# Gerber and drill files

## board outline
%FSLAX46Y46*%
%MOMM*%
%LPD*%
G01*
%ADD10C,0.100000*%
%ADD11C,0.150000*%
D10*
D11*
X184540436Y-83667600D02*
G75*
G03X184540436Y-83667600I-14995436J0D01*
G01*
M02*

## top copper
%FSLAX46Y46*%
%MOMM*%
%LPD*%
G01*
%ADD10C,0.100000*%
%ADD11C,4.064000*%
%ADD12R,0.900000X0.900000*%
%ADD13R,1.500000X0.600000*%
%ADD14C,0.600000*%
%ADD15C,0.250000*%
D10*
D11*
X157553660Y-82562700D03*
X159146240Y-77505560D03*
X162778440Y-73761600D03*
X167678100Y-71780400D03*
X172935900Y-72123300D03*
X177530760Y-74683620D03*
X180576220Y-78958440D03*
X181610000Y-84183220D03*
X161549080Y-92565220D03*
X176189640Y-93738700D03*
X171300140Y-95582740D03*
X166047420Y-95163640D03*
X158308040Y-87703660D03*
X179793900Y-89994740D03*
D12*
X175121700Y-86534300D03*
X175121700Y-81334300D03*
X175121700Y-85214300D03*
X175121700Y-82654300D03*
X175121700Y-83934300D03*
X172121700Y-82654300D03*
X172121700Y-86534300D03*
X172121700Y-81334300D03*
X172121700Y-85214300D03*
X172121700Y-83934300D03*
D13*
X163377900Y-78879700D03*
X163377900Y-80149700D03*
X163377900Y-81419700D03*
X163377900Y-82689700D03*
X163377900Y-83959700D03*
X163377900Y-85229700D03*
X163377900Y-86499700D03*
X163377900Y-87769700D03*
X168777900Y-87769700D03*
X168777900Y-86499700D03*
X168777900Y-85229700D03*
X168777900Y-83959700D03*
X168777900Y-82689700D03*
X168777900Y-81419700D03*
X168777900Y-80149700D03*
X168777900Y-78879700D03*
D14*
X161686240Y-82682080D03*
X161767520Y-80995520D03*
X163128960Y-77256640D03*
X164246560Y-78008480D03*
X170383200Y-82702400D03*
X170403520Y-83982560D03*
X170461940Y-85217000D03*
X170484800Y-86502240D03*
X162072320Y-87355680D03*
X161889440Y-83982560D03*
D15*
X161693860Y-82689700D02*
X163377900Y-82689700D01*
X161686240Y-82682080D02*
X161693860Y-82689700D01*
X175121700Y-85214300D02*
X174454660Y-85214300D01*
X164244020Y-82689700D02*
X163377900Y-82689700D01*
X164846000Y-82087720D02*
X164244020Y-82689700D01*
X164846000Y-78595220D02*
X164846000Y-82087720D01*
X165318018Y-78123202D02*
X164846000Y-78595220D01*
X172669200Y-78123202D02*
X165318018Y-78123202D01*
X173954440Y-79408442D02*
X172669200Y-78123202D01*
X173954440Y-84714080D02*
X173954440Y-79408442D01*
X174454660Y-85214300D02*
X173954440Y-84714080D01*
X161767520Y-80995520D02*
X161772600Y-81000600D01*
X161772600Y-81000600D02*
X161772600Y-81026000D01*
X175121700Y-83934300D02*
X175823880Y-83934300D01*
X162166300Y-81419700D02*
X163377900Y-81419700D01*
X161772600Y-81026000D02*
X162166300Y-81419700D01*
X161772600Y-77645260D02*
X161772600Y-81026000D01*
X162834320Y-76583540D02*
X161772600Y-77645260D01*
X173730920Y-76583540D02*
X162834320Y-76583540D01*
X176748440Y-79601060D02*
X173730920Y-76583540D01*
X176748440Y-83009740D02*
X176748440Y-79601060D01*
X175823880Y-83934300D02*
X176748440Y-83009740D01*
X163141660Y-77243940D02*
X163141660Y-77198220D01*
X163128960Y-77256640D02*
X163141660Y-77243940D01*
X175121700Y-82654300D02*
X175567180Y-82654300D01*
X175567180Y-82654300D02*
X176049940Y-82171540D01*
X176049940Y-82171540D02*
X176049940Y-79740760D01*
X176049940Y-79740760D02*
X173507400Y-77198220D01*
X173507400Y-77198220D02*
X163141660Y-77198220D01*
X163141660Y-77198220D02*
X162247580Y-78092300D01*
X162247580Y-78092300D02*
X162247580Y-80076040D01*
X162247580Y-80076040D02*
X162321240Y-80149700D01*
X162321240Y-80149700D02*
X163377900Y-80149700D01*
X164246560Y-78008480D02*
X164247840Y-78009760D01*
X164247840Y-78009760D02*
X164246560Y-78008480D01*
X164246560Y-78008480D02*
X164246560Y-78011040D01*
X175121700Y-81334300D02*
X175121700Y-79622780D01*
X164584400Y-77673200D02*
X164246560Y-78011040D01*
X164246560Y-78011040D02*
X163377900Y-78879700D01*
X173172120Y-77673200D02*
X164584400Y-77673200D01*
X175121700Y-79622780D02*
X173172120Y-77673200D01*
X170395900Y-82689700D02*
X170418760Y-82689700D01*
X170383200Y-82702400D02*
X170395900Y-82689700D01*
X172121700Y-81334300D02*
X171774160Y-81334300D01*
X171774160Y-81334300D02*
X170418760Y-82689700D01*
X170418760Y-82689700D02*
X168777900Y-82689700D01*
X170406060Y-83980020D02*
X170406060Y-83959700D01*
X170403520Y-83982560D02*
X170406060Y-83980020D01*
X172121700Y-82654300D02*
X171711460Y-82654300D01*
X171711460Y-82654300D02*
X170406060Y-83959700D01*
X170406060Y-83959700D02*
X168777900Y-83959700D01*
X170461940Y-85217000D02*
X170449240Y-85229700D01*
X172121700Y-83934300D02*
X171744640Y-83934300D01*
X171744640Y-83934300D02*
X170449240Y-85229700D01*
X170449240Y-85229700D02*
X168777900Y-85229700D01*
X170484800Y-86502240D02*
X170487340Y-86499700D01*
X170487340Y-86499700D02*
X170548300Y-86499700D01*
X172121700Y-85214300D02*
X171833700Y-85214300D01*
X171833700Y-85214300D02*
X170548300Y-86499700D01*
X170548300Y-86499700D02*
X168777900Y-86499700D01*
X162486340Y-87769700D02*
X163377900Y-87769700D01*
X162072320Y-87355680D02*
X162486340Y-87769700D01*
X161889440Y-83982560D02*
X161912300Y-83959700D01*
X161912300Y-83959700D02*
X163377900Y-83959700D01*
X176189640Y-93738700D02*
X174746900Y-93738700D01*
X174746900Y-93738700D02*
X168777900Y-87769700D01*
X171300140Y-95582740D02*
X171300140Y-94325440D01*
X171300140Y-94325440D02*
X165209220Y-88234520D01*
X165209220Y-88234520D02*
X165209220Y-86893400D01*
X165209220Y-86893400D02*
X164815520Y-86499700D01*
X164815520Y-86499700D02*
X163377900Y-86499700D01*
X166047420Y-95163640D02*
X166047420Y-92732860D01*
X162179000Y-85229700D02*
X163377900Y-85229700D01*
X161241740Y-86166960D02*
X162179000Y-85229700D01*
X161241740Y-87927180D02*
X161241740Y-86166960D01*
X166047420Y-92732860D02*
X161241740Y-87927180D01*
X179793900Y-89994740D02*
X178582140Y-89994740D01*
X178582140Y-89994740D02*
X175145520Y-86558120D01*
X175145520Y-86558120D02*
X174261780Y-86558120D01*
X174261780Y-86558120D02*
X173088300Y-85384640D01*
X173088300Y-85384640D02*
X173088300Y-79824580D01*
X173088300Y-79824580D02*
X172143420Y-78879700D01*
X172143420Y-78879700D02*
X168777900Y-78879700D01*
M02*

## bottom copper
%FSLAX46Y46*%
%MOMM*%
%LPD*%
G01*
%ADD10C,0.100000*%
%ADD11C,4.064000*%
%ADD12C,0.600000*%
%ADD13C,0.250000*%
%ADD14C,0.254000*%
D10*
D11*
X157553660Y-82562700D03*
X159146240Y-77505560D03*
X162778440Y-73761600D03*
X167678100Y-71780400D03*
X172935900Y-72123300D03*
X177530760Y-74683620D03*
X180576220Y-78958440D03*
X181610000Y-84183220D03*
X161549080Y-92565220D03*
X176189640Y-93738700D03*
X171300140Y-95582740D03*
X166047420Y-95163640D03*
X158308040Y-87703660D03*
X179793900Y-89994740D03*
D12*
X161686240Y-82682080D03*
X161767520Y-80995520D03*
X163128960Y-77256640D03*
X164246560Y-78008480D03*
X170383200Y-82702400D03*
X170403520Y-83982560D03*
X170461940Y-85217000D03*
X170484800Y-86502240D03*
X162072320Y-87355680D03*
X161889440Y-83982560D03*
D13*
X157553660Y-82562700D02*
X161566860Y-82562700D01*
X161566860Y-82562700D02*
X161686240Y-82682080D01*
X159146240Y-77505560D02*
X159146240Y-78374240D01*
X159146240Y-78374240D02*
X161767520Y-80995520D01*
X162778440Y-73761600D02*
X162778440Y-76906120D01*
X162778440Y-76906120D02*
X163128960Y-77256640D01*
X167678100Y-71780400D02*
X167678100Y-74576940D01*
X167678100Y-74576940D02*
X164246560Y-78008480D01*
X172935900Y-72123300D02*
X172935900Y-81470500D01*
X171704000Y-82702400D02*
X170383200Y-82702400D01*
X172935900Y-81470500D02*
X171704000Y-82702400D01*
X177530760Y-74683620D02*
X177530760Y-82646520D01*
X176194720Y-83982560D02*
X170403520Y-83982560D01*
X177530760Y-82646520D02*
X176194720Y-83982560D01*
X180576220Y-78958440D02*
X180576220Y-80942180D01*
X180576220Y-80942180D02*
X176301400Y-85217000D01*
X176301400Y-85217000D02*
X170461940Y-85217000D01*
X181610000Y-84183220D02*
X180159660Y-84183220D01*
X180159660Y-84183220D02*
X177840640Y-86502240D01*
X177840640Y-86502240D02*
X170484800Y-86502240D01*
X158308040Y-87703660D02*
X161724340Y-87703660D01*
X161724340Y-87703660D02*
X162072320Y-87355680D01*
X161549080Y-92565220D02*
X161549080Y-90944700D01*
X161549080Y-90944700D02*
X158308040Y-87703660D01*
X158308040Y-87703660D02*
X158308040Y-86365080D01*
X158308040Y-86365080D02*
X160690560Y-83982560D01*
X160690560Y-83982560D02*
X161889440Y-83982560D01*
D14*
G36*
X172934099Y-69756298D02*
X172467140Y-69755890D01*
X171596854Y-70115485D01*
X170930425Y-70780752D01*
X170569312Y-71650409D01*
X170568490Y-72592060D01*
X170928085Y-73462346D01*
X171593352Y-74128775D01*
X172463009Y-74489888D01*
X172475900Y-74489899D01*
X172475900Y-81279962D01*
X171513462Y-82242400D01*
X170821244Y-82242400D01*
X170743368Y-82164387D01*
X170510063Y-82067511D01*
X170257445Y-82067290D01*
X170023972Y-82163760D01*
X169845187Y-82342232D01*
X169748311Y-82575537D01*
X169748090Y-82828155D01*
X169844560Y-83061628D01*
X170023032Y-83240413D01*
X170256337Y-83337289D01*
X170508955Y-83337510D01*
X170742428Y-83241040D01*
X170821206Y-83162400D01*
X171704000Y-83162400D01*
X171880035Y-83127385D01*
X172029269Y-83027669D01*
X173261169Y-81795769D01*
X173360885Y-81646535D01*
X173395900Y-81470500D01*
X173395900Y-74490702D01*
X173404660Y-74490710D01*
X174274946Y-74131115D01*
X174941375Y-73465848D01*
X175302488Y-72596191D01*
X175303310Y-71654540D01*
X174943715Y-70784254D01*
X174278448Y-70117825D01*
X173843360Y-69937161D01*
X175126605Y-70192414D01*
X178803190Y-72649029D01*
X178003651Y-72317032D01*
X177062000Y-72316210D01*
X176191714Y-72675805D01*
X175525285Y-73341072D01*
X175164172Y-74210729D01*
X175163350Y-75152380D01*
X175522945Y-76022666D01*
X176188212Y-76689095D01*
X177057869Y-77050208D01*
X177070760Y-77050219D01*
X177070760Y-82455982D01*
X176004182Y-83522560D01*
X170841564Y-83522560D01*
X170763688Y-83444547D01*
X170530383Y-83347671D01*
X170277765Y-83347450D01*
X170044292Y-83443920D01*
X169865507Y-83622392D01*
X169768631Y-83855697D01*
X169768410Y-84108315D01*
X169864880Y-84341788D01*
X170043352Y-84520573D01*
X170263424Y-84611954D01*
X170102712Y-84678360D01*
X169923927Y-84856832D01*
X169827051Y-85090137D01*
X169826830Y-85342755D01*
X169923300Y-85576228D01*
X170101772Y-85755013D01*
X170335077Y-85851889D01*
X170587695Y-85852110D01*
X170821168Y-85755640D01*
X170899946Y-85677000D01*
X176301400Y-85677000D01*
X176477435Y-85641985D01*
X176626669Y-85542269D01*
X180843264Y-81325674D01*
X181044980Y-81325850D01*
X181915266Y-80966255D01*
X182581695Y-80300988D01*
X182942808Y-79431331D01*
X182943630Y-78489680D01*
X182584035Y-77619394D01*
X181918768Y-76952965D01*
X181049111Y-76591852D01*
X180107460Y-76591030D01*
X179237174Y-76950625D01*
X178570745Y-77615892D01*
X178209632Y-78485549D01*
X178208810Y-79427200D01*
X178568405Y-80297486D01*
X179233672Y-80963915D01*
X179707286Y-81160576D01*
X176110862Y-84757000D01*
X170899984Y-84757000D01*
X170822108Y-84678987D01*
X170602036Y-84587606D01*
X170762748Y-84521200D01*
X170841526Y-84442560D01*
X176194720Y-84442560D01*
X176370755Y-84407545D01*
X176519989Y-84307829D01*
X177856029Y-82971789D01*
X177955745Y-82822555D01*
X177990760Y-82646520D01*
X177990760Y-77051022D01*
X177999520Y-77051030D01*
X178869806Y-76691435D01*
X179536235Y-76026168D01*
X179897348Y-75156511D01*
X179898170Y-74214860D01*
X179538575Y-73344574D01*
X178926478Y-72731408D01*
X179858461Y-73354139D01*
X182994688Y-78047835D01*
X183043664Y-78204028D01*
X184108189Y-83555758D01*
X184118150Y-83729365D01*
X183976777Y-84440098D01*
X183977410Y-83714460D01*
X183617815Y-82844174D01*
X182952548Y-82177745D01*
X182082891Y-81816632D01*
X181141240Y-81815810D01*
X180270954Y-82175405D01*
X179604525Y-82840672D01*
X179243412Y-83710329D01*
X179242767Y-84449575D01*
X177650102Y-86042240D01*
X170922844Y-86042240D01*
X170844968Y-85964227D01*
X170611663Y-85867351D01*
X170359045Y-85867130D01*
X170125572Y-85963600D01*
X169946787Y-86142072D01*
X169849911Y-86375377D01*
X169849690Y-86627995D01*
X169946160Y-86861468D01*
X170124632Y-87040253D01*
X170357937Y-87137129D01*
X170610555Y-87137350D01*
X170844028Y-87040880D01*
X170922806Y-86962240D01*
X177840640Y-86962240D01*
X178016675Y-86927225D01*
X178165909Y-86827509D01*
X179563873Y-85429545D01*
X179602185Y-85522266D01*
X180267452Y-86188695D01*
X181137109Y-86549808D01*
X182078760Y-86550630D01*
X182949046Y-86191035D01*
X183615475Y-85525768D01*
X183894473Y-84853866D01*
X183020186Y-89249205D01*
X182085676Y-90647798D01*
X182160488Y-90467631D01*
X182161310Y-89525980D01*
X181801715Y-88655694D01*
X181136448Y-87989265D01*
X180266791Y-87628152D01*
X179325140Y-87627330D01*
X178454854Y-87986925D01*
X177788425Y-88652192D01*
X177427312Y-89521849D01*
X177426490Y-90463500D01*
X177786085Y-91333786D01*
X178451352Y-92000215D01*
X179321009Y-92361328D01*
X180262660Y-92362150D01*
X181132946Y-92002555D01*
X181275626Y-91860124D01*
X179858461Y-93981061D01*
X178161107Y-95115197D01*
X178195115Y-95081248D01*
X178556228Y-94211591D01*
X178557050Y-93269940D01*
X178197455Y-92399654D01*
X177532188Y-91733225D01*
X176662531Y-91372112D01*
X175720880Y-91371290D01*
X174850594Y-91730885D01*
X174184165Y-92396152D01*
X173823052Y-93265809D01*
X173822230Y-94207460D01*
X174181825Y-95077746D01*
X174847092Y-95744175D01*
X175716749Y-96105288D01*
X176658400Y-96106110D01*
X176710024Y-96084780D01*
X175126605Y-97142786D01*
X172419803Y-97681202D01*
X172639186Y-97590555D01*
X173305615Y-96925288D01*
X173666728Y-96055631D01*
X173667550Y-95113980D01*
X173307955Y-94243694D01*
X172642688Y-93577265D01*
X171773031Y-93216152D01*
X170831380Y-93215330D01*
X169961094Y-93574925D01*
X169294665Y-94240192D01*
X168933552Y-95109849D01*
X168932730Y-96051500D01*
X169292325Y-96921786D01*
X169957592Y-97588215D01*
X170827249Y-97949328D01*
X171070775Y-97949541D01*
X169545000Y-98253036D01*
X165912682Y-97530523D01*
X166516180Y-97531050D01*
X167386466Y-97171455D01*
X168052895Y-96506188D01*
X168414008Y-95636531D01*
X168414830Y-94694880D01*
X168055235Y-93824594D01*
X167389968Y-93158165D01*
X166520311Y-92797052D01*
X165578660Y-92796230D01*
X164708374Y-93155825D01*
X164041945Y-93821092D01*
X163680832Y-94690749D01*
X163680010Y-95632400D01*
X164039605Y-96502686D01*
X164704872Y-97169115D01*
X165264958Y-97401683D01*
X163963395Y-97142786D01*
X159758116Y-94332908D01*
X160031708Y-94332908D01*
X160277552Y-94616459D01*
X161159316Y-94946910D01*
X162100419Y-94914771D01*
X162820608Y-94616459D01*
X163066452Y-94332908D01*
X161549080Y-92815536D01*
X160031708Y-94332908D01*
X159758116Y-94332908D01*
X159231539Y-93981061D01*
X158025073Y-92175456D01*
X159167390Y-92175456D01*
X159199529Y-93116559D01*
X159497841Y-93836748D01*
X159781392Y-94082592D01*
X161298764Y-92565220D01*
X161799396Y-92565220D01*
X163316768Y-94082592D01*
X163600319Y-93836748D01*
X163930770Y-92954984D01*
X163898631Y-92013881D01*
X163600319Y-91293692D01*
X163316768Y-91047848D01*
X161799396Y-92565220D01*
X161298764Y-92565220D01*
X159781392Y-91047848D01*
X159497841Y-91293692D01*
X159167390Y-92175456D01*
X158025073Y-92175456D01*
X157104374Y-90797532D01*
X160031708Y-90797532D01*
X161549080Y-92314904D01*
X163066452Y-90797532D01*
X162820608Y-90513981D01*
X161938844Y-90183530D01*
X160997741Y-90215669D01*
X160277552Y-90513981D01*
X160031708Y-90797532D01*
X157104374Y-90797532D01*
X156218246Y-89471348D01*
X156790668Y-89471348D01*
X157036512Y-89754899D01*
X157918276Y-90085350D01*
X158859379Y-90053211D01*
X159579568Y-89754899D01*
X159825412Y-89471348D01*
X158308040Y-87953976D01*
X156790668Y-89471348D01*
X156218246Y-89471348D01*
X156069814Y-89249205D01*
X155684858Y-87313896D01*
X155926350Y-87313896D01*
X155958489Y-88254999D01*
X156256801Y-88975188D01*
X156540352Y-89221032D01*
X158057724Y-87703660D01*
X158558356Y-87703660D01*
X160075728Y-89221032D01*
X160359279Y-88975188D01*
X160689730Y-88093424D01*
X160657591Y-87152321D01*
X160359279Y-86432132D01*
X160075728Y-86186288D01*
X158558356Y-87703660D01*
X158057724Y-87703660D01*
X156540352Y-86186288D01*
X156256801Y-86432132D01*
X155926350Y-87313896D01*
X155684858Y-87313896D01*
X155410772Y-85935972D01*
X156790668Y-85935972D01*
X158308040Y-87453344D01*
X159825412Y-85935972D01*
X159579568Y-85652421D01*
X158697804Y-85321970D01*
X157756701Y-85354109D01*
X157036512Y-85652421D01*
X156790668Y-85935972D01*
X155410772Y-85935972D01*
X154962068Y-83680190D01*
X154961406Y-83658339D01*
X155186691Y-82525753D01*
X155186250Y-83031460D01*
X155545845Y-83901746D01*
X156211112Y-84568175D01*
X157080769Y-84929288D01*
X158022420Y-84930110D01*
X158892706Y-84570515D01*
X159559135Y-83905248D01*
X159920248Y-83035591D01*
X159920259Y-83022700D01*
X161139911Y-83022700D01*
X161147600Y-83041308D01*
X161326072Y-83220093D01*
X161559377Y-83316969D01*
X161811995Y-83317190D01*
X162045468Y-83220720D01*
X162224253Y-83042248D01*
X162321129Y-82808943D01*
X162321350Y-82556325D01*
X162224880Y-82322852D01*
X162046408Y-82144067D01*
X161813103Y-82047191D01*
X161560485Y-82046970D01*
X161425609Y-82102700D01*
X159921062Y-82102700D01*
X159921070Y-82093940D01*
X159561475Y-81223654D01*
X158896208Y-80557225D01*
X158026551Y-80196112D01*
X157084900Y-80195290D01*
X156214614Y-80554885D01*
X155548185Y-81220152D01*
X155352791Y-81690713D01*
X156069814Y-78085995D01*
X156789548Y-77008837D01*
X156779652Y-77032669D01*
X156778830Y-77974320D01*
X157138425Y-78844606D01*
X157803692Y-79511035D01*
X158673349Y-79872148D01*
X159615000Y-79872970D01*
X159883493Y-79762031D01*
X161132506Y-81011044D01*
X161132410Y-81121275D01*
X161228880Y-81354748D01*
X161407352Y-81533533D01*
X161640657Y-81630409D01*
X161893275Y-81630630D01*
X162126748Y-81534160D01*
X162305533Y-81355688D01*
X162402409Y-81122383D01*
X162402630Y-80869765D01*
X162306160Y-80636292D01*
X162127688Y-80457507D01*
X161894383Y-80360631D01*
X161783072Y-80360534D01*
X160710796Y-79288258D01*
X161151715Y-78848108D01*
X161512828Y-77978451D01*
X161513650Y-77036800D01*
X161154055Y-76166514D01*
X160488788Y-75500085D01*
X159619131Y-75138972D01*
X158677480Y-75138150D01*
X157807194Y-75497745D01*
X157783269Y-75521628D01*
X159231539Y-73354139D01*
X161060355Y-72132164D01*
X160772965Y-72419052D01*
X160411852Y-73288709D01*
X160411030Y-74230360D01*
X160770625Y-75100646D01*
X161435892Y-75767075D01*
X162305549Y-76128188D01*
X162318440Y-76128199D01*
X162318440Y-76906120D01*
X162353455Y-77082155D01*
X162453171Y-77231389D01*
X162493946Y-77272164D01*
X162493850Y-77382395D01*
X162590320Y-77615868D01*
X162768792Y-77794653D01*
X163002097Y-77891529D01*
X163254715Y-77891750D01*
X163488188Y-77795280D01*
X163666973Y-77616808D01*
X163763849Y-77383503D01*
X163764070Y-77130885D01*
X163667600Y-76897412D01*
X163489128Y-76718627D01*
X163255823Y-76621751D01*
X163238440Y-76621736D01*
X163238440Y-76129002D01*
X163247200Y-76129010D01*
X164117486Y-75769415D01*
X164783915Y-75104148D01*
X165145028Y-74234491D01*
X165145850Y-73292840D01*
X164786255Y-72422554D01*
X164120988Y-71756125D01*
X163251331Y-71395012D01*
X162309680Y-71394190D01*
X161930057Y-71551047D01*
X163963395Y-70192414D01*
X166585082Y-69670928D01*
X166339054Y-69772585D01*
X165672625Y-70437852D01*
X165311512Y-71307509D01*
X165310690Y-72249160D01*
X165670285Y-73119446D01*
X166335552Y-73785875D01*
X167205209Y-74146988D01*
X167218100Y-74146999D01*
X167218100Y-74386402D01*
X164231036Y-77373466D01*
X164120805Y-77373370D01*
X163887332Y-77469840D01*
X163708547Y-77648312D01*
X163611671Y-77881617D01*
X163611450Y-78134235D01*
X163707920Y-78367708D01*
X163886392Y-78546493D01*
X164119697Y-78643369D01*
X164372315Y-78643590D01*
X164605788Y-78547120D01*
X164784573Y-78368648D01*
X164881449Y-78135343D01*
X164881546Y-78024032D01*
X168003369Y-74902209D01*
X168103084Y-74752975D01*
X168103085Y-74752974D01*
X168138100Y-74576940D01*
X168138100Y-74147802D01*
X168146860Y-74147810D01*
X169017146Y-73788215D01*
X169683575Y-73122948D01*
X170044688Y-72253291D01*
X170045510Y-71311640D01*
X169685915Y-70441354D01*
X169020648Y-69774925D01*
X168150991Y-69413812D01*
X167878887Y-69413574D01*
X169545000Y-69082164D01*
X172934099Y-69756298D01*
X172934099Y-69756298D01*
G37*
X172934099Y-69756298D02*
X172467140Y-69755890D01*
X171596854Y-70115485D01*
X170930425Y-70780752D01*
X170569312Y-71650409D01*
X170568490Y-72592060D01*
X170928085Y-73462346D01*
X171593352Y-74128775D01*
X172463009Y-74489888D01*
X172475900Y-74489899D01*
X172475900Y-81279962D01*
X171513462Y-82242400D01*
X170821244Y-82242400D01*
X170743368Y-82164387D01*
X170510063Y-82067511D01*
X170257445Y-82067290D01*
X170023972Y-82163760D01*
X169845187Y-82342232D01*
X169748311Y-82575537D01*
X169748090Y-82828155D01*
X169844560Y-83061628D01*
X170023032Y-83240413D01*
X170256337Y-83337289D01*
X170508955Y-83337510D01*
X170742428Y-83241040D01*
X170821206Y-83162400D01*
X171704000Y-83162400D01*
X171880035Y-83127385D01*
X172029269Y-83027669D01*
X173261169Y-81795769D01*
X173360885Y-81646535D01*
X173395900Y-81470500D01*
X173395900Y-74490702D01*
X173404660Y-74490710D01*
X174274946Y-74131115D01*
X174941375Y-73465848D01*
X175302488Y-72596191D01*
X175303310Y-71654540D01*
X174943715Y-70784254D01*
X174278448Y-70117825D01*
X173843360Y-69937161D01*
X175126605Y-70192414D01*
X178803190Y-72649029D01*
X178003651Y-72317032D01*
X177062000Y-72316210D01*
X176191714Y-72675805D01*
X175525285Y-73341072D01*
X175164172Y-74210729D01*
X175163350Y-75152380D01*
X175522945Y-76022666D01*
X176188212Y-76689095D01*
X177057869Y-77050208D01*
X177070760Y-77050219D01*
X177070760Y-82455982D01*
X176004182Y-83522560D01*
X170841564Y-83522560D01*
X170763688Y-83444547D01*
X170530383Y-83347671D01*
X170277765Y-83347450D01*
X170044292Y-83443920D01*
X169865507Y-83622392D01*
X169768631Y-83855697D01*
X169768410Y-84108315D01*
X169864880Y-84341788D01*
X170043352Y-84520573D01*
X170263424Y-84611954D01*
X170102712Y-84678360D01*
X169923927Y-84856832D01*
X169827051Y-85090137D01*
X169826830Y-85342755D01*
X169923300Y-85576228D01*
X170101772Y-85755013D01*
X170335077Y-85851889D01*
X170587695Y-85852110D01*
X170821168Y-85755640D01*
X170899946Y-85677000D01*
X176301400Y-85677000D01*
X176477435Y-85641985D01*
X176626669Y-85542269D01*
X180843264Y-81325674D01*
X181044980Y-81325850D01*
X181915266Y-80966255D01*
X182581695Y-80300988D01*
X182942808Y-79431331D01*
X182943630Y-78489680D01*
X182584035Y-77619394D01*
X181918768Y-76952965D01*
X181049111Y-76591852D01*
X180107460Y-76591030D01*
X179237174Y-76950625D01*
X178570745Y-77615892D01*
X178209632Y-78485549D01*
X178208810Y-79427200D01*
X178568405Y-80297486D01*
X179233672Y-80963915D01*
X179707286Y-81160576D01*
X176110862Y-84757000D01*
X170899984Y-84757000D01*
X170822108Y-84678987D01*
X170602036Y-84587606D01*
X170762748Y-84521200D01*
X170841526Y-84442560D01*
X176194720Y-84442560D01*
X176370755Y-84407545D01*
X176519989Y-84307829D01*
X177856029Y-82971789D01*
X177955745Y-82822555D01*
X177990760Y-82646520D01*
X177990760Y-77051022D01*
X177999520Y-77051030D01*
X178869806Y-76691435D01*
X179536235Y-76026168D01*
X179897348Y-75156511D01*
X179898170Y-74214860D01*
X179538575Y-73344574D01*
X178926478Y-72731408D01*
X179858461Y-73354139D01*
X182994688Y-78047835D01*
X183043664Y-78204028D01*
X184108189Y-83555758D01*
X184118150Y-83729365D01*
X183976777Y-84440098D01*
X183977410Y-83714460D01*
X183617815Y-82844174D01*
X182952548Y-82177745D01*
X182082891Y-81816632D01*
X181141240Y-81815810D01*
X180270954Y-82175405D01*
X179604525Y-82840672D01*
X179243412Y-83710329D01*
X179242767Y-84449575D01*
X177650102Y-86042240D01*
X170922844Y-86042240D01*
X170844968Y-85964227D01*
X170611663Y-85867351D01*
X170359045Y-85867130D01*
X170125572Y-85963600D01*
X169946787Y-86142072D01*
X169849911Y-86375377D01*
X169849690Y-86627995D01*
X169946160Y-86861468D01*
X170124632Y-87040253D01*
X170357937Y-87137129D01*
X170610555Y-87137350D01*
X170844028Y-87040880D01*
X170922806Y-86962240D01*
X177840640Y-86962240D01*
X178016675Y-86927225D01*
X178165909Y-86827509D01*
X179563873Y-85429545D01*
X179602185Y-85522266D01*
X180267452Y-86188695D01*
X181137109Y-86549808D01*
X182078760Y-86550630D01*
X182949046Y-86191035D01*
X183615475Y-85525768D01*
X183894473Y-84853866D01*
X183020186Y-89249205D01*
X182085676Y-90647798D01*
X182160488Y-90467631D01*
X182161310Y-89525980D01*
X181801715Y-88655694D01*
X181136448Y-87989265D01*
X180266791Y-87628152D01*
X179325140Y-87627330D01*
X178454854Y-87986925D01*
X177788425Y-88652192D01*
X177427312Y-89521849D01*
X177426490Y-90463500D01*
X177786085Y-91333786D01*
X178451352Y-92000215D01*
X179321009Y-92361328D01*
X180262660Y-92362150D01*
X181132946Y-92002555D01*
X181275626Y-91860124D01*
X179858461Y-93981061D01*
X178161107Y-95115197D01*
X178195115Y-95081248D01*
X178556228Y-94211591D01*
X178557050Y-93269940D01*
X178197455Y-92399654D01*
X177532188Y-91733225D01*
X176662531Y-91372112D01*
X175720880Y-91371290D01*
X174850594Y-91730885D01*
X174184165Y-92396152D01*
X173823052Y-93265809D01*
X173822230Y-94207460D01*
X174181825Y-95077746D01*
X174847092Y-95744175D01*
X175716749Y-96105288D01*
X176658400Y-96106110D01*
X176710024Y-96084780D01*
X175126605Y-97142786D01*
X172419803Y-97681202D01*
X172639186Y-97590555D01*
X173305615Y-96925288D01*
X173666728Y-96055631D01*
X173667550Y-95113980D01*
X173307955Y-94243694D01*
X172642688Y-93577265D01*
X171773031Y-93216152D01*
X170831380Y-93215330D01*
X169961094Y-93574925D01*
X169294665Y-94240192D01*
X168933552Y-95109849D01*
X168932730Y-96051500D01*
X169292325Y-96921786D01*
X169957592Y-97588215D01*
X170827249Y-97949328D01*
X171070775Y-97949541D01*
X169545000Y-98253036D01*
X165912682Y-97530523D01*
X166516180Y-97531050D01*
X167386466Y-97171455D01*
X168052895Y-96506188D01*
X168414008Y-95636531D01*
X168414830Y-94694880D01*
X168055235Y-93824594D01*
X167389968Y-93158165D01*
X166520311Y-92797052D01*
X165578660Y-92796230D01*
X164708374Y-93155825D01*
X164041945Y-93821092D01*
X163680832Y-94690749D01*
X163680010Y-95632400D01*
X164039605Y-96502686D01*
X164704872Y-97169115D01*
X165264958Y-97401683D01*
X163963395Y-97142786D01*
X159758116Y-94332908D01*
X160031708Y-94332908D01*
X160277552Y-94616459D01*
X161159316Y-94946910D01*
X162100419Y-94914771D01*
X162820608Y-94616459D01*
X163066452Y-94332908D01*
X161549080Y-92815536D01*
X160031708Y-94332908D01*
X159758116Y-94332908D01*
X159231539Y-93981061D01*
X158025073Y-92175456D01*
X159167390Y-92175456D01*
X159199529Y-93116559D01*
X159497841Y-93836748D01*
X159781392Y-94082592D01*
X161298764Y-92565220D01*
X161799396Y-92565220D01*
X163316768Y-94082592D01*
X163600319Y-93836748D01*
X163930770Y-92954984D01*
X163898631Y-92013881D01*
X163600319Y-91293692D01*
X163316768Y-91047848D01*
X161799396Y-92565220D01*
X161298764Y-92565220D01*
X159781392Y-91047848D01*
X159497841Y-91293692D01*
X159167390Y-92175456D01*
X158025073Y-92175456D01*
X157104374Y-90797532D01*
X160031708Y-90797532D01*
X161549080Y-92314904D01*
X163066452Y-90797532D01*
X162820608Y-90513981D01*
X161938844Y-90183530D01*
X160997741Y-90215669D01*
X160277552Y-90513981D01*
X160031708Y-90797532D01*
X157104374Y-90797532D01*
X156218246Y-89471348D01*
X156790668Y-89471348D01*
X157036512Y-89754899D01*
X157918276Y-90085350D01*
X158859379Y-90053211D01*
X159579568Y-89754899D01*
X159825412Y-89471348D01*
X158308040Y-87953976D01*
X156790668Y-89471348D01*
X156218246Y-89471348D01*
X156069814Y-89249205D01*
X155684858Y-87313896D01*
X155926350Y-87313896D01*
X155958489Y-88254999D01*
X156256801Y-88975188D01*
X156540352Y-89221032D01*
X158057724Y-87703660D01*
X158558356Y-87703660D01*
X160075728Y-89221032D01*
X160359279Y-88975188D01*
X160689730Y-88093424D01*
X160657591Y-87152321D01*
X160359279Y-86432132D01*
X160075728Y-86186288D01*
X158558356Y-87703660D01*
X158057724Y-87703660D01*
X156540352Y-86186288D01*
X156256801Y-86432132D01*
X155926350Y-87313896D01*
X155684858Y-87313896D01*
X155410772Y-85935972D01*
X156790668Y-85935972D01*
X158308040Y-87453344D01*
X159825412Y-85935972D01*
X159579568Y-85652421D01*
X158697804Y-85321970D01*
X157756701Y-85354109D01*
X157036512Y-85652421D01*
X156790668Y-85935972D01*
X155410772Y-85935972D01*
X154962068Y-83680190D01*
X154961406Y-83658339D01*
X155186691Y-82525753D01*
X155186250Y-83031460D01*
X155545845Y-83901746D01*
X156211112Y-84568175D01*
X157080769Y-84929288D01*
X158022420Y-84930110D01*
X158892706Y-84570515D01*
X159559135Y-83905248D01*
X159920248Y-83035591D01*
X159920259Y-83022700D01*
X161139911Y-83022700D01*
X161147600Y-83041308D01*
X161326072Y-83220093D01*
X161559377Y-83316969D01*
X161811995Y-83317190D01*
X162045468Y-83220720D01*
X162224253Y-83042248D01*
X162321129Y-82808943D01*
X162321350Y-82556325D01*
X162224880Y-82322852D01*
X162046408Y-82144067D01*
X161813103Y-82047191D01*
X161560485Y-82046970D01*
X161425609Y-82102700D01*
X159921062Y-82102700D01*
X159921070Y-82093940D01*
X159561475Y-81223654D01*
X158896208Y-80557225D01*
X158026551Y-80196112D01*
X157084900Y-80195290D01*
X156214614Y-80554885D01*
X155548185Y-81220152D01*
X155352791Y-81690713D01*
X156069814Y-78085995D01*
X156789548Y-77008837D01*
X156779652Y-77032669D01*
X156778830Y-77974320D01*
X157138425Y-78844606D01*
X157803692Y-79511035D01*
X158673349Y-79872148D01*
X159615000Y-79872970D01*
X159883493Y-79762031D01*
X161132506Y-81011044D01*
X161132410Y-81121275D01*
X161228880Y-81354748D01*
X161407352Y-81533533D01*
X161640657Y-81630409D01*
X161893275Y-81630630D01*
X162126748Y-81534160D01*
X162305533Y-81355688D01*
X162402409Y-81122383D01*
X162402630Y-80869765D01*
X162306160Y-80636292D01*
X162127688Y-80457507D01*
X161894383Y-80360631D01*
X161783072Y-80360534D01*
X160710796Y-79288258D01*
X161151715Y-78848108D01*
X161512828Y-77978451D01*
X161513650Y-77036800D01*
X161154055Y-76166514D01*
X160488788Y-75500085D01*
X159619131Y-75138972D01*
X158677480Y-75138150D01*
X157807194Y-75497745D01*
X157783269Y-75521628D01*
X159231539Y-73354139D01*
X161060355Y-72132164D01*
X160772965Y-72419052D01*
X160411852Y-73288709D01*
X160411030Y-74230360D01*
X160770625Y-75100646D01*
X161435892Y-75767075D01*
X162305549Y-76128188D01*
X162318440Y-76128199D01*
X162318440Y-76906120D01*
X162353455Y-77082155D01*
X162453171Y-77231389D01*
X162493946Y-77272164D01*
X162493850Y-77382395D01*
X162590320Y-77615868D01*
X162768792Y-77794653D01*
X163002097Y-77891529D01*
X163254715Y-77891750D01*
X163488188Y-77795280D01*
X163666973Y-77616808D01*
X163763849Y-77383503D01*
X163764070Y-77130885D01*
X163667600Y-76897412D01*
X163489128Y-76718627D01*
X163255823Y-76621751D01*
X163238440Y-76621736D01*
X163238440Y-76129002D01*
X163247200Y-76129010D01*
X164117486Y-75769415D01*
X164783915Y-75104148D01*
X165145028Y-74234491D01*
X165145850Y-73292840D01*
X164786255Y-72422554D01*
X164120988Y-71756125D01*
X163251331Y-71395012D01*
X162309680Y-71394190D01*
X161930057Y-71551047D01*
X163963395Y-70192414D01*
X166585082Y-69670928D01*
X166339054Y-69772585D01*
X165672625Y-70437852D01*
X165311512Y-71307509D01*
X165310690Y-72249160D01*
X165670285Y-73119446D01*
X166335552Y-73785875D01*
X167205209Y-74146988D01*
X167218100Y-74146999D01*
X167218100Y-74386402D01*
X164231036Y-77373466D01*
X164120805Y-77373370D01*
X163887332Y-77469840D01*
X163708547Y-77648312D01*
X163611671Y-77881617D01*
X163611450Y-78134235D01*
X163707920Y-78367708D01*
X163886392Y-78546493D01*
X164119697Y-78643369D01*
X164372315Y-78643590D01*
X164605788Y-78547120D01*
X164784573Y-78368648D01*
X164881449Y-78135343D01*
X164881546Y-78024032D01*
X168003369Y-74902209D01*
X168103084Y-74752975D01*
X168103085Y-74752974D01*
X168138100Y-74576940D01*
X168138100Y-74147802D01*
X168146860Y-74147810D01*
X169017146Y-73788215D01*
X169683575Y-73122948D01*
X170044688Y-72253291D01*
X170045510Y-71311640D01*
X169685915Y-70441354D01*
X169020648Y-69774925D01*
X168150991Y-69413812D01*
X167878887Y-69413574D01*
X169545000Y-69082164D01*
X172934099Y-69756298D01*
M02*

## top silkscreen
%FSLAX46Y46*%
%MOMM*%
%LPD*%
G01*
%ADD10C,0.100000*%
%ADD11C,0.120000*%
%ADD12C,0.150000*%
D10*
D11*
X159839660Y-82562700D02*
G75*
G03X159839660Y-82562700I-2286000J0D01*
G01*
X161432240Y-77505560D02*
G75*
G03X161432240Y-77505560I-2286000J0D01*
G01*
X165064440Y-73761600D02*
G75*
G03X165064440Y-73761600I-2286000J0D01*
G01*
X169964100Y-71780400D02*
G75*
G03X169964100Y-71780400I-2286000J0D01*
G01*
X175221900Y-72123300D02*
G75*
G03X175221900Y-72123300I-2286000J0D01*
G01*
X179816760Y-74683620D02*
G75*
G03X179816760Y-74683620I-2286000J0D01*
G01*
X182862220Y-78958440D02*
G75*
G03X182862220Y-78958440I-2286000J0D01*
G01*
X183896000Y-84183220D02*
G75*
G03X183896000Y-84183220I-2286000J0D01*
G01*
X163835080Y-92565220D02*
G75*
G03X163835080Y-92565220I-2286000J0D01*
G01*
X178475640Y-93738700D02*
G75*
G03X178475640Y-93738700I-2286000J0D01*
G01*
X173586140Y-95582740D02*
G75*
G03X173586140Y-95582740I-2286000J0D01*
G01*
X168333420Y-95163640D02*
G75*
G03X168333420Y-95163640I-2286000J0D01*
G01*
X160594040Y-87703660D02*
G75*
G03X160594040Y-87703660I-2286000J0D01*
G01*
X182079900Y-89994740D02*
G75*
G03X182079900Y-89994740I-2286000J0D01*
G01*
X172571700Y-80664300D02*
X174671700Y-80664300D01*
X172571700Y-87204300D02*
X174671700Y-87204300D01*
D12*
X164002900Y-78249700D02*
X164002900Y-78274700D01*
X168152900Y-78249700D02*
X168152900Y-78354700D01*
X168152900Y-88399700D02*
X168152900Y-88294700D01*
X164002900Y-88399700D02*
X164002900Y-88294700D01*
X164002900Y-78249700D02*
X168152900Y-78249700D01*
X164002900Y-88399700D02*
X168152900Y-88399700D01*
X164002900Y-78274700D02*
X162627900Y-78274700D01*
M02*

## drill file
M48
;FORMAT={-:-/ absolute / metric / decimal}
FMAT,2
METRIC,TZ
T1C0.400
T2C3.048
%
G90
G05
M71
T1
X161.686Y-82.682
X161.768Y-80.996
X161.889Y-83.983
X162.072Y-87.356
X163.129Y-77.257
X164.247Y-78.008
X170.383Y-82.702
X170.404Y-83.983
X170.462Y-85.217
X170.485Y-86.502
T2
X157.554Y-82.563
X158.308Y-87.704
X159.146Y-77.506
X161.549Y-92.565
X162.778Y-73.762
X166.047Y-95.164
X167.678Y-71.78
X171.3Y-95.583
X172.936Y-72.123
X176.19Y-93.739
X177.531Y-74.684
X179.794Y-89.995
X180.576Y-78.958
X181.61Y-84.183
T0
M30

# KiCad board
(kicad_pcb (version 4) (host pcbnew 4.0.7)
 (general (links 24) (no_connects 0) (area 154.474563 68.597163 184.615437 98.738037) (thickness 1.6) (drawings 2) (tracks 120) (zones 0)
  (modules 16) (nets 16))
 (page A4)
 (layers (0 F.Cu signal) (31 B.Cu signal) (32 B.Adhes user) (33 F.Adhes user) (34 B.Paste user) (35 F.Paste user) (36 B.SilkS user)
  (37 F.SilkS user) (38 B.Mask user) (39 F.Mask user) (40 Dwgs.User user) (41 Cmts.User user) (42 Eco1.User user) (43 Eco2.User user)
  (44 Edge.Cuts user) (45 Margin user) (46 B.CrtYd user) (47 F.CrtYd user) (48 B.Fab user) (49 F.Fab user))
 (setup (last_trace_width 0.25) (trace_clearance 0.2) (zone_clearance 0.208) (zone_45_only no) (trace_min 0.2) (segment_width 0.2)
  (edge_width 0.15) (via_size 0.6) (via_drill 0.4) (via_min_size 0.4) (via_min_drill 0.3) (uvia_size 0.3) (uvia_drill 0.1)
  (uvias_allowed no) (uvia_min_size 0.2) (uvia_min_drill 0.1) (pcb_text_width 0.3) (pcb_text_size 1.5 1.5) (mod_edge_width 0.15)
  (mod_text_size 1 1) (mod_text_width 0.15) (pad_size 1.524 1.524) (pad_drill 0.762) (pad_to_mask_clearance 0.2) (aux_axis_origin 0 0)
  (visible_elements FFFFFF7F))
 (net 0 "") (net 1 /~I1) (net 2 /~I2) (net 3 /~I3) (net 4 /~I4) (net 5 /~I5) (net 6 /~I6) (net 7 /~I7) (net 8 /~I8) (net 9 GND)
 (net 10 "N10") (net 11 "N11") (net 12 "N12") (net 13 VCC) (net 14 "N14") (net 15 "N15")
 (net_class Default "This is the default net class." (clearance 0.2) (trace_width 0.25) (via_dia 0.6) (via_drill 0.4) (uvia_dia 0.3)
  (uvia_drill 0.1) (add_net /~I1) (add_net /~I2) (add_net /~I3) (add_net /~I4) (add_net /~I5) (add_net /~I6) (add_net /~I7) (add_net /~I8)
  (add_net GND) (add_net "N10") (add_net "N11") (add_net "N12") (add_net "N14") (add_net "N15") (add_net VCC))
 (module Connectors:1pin (layer F.Cu) (at 157.55366 82.5627)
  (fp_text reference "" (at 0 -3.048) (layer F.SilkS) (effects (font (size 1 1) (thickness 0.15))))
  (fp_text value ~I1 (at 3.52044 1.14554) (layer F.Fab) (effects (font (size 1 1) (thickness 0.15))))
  (fp_circle (center 0 0) (end 0 -2.286) (layer F.SilkS) (width 0.12))
  (pad 1 thru_hole circle (at 0 0) (size 4.064 4.064) (drill 3.048) (layers *.Cu *.Mask) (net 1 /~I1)))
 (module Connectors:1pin (layer F.Cu) (at 159.14624 77.50556)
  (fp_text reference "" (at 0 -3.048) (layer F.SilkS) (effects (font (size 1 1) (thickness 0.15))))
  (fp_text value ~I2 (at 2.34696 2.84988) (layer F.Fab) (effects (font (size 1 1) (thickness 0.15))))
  (fp_circle (center 0 0) (end 0 -2.286) (layer F.SilkS) (width 0.12))
  (pad 1 thru_hole circle (at 0 0) (size 4.064 4.064) (drill 3.048) (layers *.Cu *.Mask) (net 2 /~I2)))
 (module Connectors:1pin (layer F.Cu) (at 162.77844 73.7616)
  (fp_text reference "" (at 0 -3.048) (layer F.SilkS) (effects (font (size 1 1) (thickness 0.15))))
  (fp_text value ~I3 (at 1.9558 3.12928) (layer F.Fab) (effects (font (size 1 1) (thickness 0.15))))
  (fp_circle (center 0 0) (end 0 -2.286) (layer F.SilkS) (width 0.12))
  (pad 1 thru_hole circle (at 0 0) (size 4.064 4.064) (drill 3.048) (layers *.Cu *.Mask) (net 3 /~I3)))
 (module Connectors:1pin (layer F.Cu) (at 167.6781 71.7804)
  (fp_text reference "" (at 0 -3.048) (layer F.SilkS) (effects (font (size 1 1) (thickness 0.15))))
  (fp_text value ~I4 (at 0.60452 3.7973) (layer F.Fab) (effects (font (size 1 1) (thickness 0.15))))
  (fp_circle (center 0 0) (end 0 -2.286) (layer F.SilkS) (width 0.12))
  (pad 1 thru_hole circle (at 0 0) (size 4.064 4.064) (drill 3.048) (layers *.Cu *.Mask) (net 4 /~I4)))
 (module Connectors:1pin (layer F.Cu) (at 172.9359 72.1233)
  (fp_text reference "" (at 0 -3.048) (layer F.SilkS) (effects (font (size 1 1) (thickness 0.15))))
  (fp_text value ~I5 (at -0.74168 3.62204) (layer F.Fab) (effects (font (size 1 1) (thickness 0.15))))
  (fp_circle (center 0 0) (end 0 -2.286) (layer F.SilkS) (width 0.12))
  (pad 1 thru_hole circle (at 0 0) (size 4.064 4.064) (drill 3.048) (layers *.Cu *.Mask) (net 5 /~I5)))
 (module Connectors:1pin (layer F.Cu) (at 177.53076 74.68362)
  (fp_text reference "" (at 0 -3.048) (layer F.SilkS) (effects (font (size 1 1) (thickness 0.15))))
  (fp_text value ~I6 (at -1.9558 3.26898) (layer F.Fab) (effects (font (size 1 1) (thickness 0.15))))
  (fp_circle (center 0 0) (end 0 -2.286) (layer F.SilkS) (width 0.12))
  (pad 1 thru_hole circle (at 0 0) (size 4.064 4.064) (drill 3.048) (layers *.Cu *.Mask) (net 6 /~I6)))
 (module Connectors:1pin (layer F.Cu) (at 180.57622 78.95844)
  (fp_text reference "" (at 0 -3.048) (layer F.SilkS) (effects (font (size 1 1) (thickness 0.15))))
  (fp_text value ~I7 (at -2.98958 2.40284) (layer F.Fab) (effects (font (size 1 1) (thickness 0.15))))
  (fp_circle (center 0 0) (end 0 -2.286) (layer F.SilkS) (width 0.12))
  (pad 1 thru_hole circle (at 0 0) (size 4.064 4.064) (drill 3.048) (layers *.Cu *.Mask) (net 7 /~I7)))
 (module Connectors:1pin (layer F.Cu) (at 181.61 84.18322)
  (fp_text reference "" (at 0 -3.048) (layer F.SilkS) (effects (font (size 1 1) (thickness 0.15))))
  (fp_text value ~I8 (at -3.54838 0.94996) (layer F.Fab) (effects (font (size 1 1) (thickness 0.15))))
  (fp_circle (center 0 0) (end 0 -2.286) (layer F.SilkS) (width 0.12))
  (pad 1 thru_hole circle (at 0 0) (size 4.064 4.064) (drill 3.048) (layers *.Cu *.Mask) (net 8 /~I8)))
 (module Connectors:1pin (layer F.Cu) (at 161.54908 92.56522)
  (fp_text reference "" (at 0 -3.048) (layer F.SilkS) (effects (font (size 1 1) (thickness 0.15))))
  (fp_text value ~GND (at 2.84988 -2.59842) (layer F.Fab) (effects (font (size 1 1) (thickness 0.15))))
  (fp_circle (center 0 0) (end 0 -2.286) (layer F.SilkS) (width 0.12))
  (pad 1 thru_hole circle (at 0 0) (size 4.064 4.064) (drill 3.048) (layers *.Cu *.Mask) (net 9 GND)))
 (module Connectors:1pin (layer F.Cu) (at 176.18964 93.7387)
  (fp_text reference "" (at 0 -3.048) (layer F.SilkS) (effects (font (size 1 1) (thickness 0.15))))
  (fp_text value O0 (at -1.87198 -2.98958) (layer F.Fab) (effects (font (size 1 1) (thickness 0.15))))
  (fp_circle (center 0 0) (end 0 -2.286) (layer F.SilkS) (width 0.12))
  (pad 1 thru_hole circle (at 0 0) (size 4.064 4.064) (drill 3.048) (layers *.Cu *.Mask) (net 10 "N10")))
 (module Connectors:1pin (layer F.Cu) (at 171.30014 95.58274)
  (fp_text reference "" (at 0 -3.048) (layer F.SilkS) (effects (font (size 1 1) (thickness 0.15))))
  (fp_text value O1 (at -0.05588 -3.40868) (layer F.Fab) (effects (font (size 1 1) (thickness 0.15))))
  (fp_circle (center 0 0) (end 0 -2.286) (layer F.SilkS) (width 0.12))
  (pad 1 thru_hole circle (at 0 0) (size 4.064 4.064) (drill 3.048) (layers *.Cu *.Mask) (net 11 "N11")))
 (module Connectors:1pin (layer F.Cu) (at 166.04742 95.16364)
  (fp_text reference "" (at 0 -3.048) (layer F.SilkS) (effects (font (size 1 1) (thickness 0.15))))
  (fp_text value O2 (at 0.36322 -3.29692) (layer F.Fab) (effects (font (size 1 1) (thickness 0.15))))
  (fp_circle (center 0 0) (end 0 -2.286) (layer F.SilkS) (width 0.12))
  (pad 1 thru_hole circle (at 0 0) (size 4.064 4.064) (drill 3.048) (layers *.Cu *.Mask) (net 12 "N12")))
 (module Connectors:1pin (layer F.Cu) (at 158.30804 87.70366)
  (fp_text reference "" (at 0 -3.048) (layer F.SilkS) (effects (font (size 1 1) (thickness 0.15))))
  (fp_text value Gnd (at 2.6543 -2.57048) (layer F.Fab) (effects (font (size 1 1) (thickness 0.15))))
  (fp_circle (center 0 0) (end 0 -2.286) (layer F.SilkS) (width 0.12))
  (pad 1 thru_hole circle (at 0 0) (size 4.064 4.064) (drill 3.048) (layers *.Cu *.Mask) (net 9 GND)))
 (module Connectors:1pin (layer F.Cu) (at 179.7939 89.99474)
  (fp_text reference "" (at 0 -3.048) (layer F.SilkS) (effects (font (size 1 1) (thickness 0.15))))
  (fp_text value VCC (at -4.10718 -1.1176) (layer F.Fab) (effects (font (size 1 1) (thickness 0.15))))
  (fp_circle (center 0 0) (end 0 -2.286) (layer F.SilkS) (width 0.12))
  (pad 1 thru_hole circle (at 0 0) (size 4.064 4.064) (drill 3.048) (layers *.Cu *.Mask) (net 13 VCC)))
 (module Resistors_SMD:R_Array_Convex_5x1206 (layer F.Cu) (at 173.6217 83.9343 180)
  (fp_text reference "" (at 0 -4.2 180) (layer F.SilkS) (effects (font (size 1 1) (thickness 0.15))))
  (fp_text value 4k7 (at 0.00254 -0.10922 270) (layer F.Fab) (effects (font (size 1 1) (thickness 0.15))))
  (fp_line (start 1.05 3.27) (end -1.05 3.27) (layer F.SilkS) (width 0.12))
  (fp_line (start 1.05 -3.27) (end -1.05 -3.27) (layer F.SilkS) (width 0.12))
  (pad 1 smd rect (at -1.5 -2.6 180) (size 0.9 0.9) (layers F.Cu F.Paste F.Mask) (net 13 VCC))
  (pad 5 smd rect (at -1.5 2.6 180) (size 0.9 0.9) (layers F.Cu F.Paste F.Mask) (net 4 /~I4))
  (pad 2 smd rect (at -1.5 -1.28 180) (size 0.9 0.9) (layers F.Cu F.Paste F.Mask) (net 1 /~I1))
  (pad 4 smd rect (at -1.5 1.28 180) (size 0.9 0.9) (layers F.Cu F.Paste F.Mask) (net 3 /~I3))
  (pad 3 smd rect (at -1.5 0 180) (size 0.9 0.9) (layers F.Cu F.Paste F.Mask) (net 2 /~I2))
  (pad 7 smd rect (at 1.5 1.28 180) (size 0.9 0.9) (layers F.Cu F.Paste F.Mask) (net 6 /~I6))
  (pad 10 smd rect (at 1.5 -2.6 180) (size 0.9 0.9) (layers F.Cu F.Paste F.Mask))
  (pad 6 smd rect (at 1.5 2.6 180) (size 0.9 0.9) (layers F.Cu F.Paste F.Mask) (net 5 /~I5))
  (pad 9 smd rect (at 1.5 -1.28 180) (size 0.9 0.9) (layers F.Cu F.Paste F.Mask) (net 8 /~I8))
  (pad 8 smd rect (at 1.5 0 180) (size 0.9 0.9) (layers F.Cu F.Paste F.Mask) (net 7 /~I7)))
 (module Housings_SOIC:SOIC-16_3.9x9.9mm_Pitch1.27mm (layer F.Cu) (at 166.0779 83.3247)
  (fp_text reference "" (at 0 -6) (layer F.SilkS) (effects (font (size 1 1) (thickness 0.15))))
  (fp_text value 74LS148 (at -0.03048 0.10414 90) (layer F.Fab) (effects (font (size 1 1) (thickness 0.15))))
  (fp_line (start -2.075 -5.075) (end -2.075 -5.05) (layer F.SilkS) (width 0.15))
  (fp_line (start 2.075 -5.075) (end 2.075 -4.97) (layer F.SilkS) (width 0.15))
  (fp_line (start 2.075 5.075) (end 2.075 4.97) (layer F.SilkS) (width 0.15))
  (fp_line (start -2.075 5.075) (end -2.075 4.97) (layer F.SilkS) (width 0.15))
  (fp_line (start -2.075 -5.075) (end 2.075 -5.075) (layer F.SilkS) (width 0.15))
  (fp_line (start -2.075 5.075) (end 2.075 5.075) (layer F.SilkS) (width 0.15))
  (fp_line (start -2.075 -5.05) (end -3.45 -5.05) (layer F.SilkS) (width 0.15))
  (pad 1 smd rect (at -2.7 -4.445) (size 1.5 0.6) (layers F.Cu F.Paste F.Mask) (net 4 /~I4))
  (pad 2 smd rect (at -2.7 -3.175) (size 1.5 0.6) (layers F.Cu F.Paste F.Mask) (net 3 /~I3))
  (pad 3 smd rect (at -2.7 -1.905) (size 1.5 0.6) (layers F.Cu F.Paste F.Mask) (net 2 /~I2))
  (pad 4 smd rect (at -2.7 -0.635) (size 1.5 0.6) (layers F.Cu F.Paste F.Mask) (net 1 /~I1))
  (pad 5 smd rect (at -2.7 0.635) (size 1.5 0.6) (layers F.Cu F.Paste F.Mask) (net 9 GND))
  (pad 6 smd rect (at -2.7 1.905) (size 1.5 0.6) (layers F.Cu F.Paste F.Mask) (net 12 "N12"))
  (pad 7 smd rect (at -2.7 3.175) (size 1.5 0.6) (layers F.Cu F.Paste F.Mask) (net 11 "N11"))
  (pad 8 smd rect (at -2.7 4.445) (size 1.5 0.6) (layers F.Cu F.Paste F.Mask) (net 9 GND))
  (pad 9 smd rect (at 2.7 4.445) (size 1.5 0.6) (layers F.Cu F.Paste F.Mask) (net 10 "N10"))
  (pad 10 smd rect (at 2.7 3.175) (size 1.5 0.6) (layers F.Cu F.Paste F.Mask) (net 8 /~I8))
  (pad 11 smd rect (at 2.7 1.905) (size 1.5 0.6) (layers F.Cu F.Paste F.Mask) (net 7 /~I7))
  (pad 12 smd rect (at 2.7 0.635) (size 1.5 0.6) (layers F.Cu F.Paste F.Mask) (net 6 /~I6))
  (pad 13 smd rect (at 2.7 -0.635) (size 1.5 0.6) (layers F.Cu F.Paste F.Mask) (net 5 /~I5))
  (pad 14 smd rect (at 2.7 -1.905) (size 1.5 0.6) (layers F.Cu F.Paste F.Mask) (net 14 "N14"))
  (pad 15 smd rect (at 2.7 -3.175) (size 1.5 0.6) (layers F.Cu F.Paste F.Mask) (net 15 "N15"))
  (pad 16 smd rect (at 2.7 -4.445) (size 1.5 0.6) (layers F.Cu F.Paste F.Mask) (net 13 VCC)))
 (gr_circle (center 169.545 83.6676) (end 180.6321 93.7641) (layer Edge.Cuts) (width 0.15))
 (segment (start 157.55366 82.5627) (end 161.56686 82.5627) (width 0.25) (layer B.Cu) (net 1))
 (segment (start 161.69386 82.6897) (end 163.3779 82.6897) (width 0.25) (layer F.Cu) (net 1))
 (segment (start 161.68624 82.68208) (end 161.69386 82.6897) (width 0.25) (layer F.Cu) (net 1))
 (via (at 161.68624 82.68208) (size 0.6) (drill 0.4) (layers F.Cu B.Cu) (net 1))
 (segment (start 161.56686 82.5627) (end 161.68624 82.68208) (width 0.25) (layer B.Cu) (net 1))
 (segment (start 175.1217 85.2143) (end 174.45466 85.2143) (width 0.25) (layer F.Cu) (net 1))
 (segment (start 164.24402 82.6897) (end 163.3779 82.6897) (width 0.25) (layer F.Cu) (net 1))
 (segment (start 164.846 82.08772) (end 164.24402 82.6897) (width 0.25) (layer F.Cu) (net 1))
 (segment (start 164.846 78.59522) (end 164.846 82.08772) (width 0.25) (layer F.Cu) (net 1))
 (segment (start 165.318018 78.123202) (end 164.846 78.59522) (width 0.25) (layer F.Cu) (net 1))
 (segment (start 172.6692 78.123202) (end 165.318018 78.123202) (width 0.25) (layer F.Cu) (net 1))
 (segment (start 173.95444 79.408442) (end 172.6692 78.123202) (width 0.25) (layer F.Cu) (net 1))
 (segment (start 173.95444 84.71408) (end 173.95444 79.408442) (width 0.25) (layer F.Cu) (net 1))
 (segment (start 174.45466 85.2143) (end 173.95444 84.71408) (width 0.25) (layer F.Cu) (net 1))
 (segment (start 159.14624 77.50556) (end 159.14624 78.37424) (width 0.25) (layer B.Cu) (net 2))
 (segment (start 159.14624 78.37424) (end 161.76752 80.99552) (width 0.25) (layer B.Cu) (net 2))
 (via (at 161.76752 80.99552) (size 0.6) (drill 0.4) (layers F.Cu B.Cu) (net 2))
 (segment (start 161.76752 80.99552) (end 161.7726 81.0006) (width 0.25) (layer F.Cu) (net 2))
 (segment (start 161.7726 81.0006) (end 161.7726 81.026) (width 0.25) (layer F.Cu) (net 2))
 (segment (start 175.1217 83.9343) (end 175.82388 83.9343) (width 0.25) (layer F.Cu) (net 2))
 (segment (start 162.1663 81.4197) (end 163.3779 81.4197) (width 0.25) (layer F.Cu) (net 2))
 (segment (start 161.7726 81.026) (end 162.1663 81.4197) (width 0.25) (layer F.Cu) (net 2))
 (segment (start 161.7726 77.64526) (end 161.7726 81.026) (width 0.25) (layer F.Cu) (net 2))
 (segment (start 162.83432 76.58354) (end 161.7726 77.64526) (width 0.25) (layer F.Cu) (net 2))
 (segment (start 173.73092 76.58354) (end 162.83432 76.58354) (width 0.25) (layer F.Cu) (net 2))
 (segment (start 176.74844 79.60106) (end 173.73092 76.58354) (width 0.25) (layer F.Cu) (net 2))
 (segment (start 176.74844 83.00974) (end 176.74844 79.60106) (width 0.25) (layer F.Cu) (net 2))
 (segment (start 175.82388 83.9343) (end 176.74844 83.00974) (width 0.25) (layer F.Cu) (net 2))
 (segment (start 162.77844 73.7616) (end 162.77844 76.90612) (width 0.25) (layer B.Cu) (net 3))
 (segment (start 163.14166 77.24394) (end 163.14166 77.19822) (width 0.25) (layer F.Cu) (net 3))
 (segment (start 163.12896 77.25664) (end 163.14166 77.24394) (width 0.25) (layer F.Cu) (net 3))
 (via (at 163.12896 77.25664) (size 0.6) (drill 0.4) (layers F.Cu B.Cu) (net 3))
 (segment (start 162.77844 76.90612) (end 163.12896 77.25664) (width 0.25) (layer B.Cu) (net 3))
 (segment (start 175.1217 82.6543) (end 175.56718 82.6543) (width 0.25) (layer F.Cu) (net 3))
 (segment (start 175.56718 82.6543) (end 176.04994 82.17154) (width 0.25) (layer F.Cu) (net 3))
 (segment (start 176.04994 82.17154) (end 176.04994 79.74076) (width 0.25) (layer F.Cu) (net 3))
 (segment (start 176.04994 79.74076) (end 173.5074 77.19822) (width 0.25) (layer F.Cu) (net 3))
 (segment (start 173.5074 77.19822) (end 163.14166 77.19822) (width 0.25) (layer F.Cu) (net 3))
 (segment (start 163.14166 77.19822) (end 162.24758 78.0923) (width 0.25) (layer F.Cu) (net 3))
 (segment (start 162.24758 78.0923) (end 162.24758 80.07604) (width 0.25) (layer F.Cu) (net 3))
 (segment (start 162.24758 80.07604) (end 162.32124 80.1497) (width 0.25) (layer F.Cu) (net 3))
 (segment (start 162.32124 80.1497) (end 163.3779 80.1497) (width 0.25) (layer F.Cu) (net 3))
 (segment (start 167.6781 71.7804) (end 167.6781 74.57694) (width 0.25) (layer B.Cu) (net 4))
 (via (at 164.24656 78.00848) (size 0.6) (drill 0.4) (layers F.Cu B.Cu) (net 4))
 (segment (start 167.6781 74.57694) (end 164.24656 78.00848) (width 0.25) (layer B.Cu) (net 4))
 (segment (start 164.24656 78.00848) (end 164.24784 78.00976) (width 0.25) (layer F.Cu) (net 4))
 (segment (start 164.24784 78.00976) (end 164.24656 78.00848) (width 0.25) (layer F.Cu) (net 4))
 (segment (start 164.24656 78.00848) (end 164.24656 78.01104) (width 0.25) (layer F.Cu) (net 4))
 (segment (start 175.1217 81.3343) (end 175.1217 79.62278) (width 0.25) (layer F.Cu) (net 4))
 (segment (start 164.5844 77.6732) (end 164.24656 78.01104) (width 0.25) (layer F.Cu) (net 4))
 (segment (start 164.24656 78.01104) (end 163.3779 78.8797) (width 0.25) (layer F.Cu) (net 4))
 (segment (start 173.17212 77.6732) (end 164.5844 77.6732) (width 0.25) (layer F.Cu) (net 4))
 (segment (start 175.1217 79.62278) (end 173.17212 77.6732) (width 0.25) (layer F.Cu) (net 4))
 (segment (start 172.9359 72.1233) (end 172.9359 81.4705) (width 0.25) (layer B.Cu) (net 5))
 (segment (start 170.3959 82.6897) (end 170.41876 82.6897) (width 0.25) (layer F.Cu) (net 5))
 (segment (start 170.3832 82.7024) (end 170.3959 82.6897) (width 0.25) (layer F.Cu) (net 5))
 (via (at 170.3832 82.7024) (size 0.6) (drill 0.4) (layers F.Cu B.Cu) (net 5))
 (segment (start 171.704 82.7024) (end 170.3832 82.7024) (width 0.25) (layer B.Cu) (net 5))
 (segment (start 172.9359 81.4705) (end 171.704 82.7024) (width 0.25) (layer B.Cu) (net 5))
 (segment (start 172.1217 81.3343) (end 171.77416 81.3343) (width 0.25) (layer F.Cu) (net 5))
 (segment (start 171.77416 81.3343) (end 170.41876 82.6897) (width 0.25) (layer F.Cu) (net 5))
 (segment (start 170.41876 82.6897) (end 168.7779 82.6897) (width 0.25) (layer F.Cu) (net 5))
 (segment (start 177.53076 74.68362) (end 177.53076 82.64652) (width 0.25) (layer B.Cu) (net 6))
 (segment (start 170.40606 83.98002) (end 170.40606 83.9597) (width 0.25) (layer F.Cu) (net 6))
 (segment (start 170.40352 83.98256) (end 170.40606 83.98002) (width 0.25) (layer F.Cu) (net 6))
 (via (at 170.40352 83.98256) (size 0.6) (drill 0.4) (layers F.Cu B.Cu) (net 6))
 (segment (start 176.19472 83.98256) (end 170.40352 83.98256) (width 0.25) (layer B.Cu) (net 6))
 (segment (start 177.53076 82.64652) (end 176.19472 83.98256) (width 0.25) (layer B.Cu) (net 6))
 (segment (start 172.1217 82.6543) (end 171.71146 82.6543) (width 0.25) (layer F.Cu) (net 6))
 (segment (start 171.71146 82.6543) (end 170.40606 83.9597) (width 0.25) (layer F.Cu) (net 6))
 (segment (start 170.40606 83.9597) (end 168.7779 83.9597) (width 0.25) (layer F.Cu) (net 6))
 (segment (start 180.57622 78.95844) (end 180.57622 80.94218) (width 0.25) (layer B.Cu) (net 7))
 (segment (start 180.57622 80.94218) (end 176.3014 85.217) (width 0.25) (layer B.Cu) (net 7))
 (segment (start 176.3014 85.217) (end 170.46194 85.217) (width 0.25) (layer B.Cu) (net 7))
 (via (at 170.46194 85.217) (size 0.6) (drill 0.4) (layers F.Cu B.Cu) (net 7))
 (segment (start 170.46194 85.217) (end 170.44924 85.2297) (width 0.25) (layer F.Cu) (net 7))
 (segment (start 172.1217 83.9343) (end 171.74464 83.9343) (width 0.25) (layer F.Cu) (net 7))
 (segment (start 171.74464 83.9343) (end 170.44924 85.2297) (width 0.25) (layer F.Cu) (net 7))
 (segment (start 170.44924 85.2297) (end 168.7779 85.2297) (width 0.25) (layer F.Cu) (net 7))
 (segment (start 181.61 84.18322) (end 180.15966 84.18322) (width 0.25) (layer B.Cu) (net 8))
 (segment (start 180.15966 84.18322) (end 177.84064 86.50224) (width 0.25) (layer B.Cu) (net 8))
 (segment (start 177.84064 86.50224) (end 170.4848 86.50224) (width 0.25) (layer B.Cu) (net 8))
 (via (at 170.4848 86.50224) (size 0.6) (drill 0.4) (layers F.Cu B.Cu) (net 8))
 (segment (start 170.4848 86.50224) (end 170.48734 86.4997) (width 0.25) (layer F.Cu) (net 8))
 (segment (start 170.48734 86.4997) (end 170.5483 86.4997) (width 0.25) (layer F.Cu) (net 8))
 (segment (start 172.1217 85.2143) (end 171.8337 85.2143) (width 0.25) (layer F.Cu) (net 8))
 (segment (start 171.8337 85.2143) (end 170.5483 86.4997) (width 0.25) (layer F.Cu) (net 8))
 (segment (start 170.5483 86.4997) (end 168.7779 86.4997) (width 0.25) (layer F.Cu) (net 8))
 (segment (start 158.30804 87.70366) (end 161.72434 87.70366) (width 0.25) (layer B.Cu) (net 9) (status 400000))
 (segment (start 162.48634 87.7697) (end 163.3779 87.7697) (width 0.25) (layer F.Cu) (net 9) (status 800000))
 (segment (start 162.07232 87.35568) (end 162.48634 87.7697) (width 0.25) (layer F.Cu) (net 9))
 (via (at 162.07232 87.35568) (size 0.6) (drill 0.4) (layers F.Cu B.Cu) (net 9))
 (segment (start 161.72434 87.70366) (end 162.07232 87.35568) (width 0.25) (layer B.Cu) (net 9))
 (segment (start 161.54908 92.56522) (end 161.54908 90.9447) (width 0.25) (layer B.Cu) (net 9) (status C00000))
 (segment (start 161.54908 90.9447) (end 158.30804 87.70366) (width 0.25) (layer B.Cu) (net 9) (status C00000))
 (segment (start 158.30804 87.70366) (end 158.30804 86.36508) (width 0.25) (layer B.Cu) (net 9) (status C00000))
 (segment (start 158.30804 86.36508) (end 160.69056 83.98256) (width 0.25) (layer B.Cu) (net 9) (status 400000))
 (segment (start 160.69056 83.98256) (end 161.88944 83.98256) (width 0.25) (layer B.Cu) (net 9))
 (via (at 161.88944 83.98256) (size 0.6) (drill 0.4) (layers F.Cu B.Cu) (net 9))
 (segment (start 161.88944 83.98256) (end 161.9123 83.9597) (width 0.25) (layer F.Cu) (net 9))
 (segment (start 161.9123 83.9597) (end 163.3779 83.9597) (width 0.25) (layer F.Cu) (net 9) (status 800000))
 (segment (start 176.18964 93.7387) (end 174.7469 93.7387) (width 0.25) (layer F.Cu) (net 10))
 (segment (start 174.7469 93.7387) (end 168.7779 87.7697) (width 0.25) (layer F.Cu) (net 10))
 (segment (start 171.30014 95.58274) (end 171.30014 94.32544) (width 0.25) (layer F.Cu) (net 11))
 (segment (start 171.30014 94.32544) (end 165.20922 88.23452) (width 0.25) (layer F.Cu) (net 11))
 (segment (start 165.20922 88.23452) (end 165.20922 86.8934) (width 0.25) (layer F.Cu) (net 11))
 (segment (start 165.20922 86.8934) (end 164.81552 86.4997) (width 0.25) (layer F.Cu) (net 11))
 (segment (start 164.81552 86.4997) (end 163.3779 86.4997) (width 0.25) (layer F.Cu) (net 11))
 (segment (start 166.04742 95.16364) (end 166.04742 92.73286) (width 0.25) (layer F.Cu) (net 12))
 (segment (start 162.179 85.2297) (end 163.3779 85.2297) (width 0.25) (layer F.Cu) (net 12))
 (segment (start 161.24174 86.16696) (end 162.179 85.2297) (width 0.25) (layer F.Cu) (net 12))
 (segment (start 161.24174 87.92718) (end 161.24174 86.16696) (width 0.25) (layer F.Cu) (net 12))
 (segment (start 166.04742 92.73286) (end 161.24174 87.92718) (width 0.25) (layer F.Cu) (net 12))
 (segment (start 179.7939 89.99474) (end 178.58214 89.99474) (width 0.25) (layer F.Cu) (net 13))
 (segment (start 178.58214 89.99474) (end 175.14552 86.55812) (width 0.25) (layer F.Cu) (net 13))
 (segment (start 175.14552 86.55812) (end 174.26178 86.55812) (width 0.25) (layer F.Cu) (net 13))
 (segment (start 174.26178 86.55812) (end 173.0883 85.38464) (width 0.25) (layer F.Cu) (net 13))
 (segment (start 173.0883 85.38464) (end 173.0883 79.82458) (width 0.25) (layer F.Cu) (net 13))
 (segment (start 173.0883 79.82458) (end 172.14342 78.8797) (width 0.25) (layer F.Cu) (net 13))
 (segment (start 172.14342 78.8797) (end 168.7779 78.8797) (width 0.25) (layer F.Cu) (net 13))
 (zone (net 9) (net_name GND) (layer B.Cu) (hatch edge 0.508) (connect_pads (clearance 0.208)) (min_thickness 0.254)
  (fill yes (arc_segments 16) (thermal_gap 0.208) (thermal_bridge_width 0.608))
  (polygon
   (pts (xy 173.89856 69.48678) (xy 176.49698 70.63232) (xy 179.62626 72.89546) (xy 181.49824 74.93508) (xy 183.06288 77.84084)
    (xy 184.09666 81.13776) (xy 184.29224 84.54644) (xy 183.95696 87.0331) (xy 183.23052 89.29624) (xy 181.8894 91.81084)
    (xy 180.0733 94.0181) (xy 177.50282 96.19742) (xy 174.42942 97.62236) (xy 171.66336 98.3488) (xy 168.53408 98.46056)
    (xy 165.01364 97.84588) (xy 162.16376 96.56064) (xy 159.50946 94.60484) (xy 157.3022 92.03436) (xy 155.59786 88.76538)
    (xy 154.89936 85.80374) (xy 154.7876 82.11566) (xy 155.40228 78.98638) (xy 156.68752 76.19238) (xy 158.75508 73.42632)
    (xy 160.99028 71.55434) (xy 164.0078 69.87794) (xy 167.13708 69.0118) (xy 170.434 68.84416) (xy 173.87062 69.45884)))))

